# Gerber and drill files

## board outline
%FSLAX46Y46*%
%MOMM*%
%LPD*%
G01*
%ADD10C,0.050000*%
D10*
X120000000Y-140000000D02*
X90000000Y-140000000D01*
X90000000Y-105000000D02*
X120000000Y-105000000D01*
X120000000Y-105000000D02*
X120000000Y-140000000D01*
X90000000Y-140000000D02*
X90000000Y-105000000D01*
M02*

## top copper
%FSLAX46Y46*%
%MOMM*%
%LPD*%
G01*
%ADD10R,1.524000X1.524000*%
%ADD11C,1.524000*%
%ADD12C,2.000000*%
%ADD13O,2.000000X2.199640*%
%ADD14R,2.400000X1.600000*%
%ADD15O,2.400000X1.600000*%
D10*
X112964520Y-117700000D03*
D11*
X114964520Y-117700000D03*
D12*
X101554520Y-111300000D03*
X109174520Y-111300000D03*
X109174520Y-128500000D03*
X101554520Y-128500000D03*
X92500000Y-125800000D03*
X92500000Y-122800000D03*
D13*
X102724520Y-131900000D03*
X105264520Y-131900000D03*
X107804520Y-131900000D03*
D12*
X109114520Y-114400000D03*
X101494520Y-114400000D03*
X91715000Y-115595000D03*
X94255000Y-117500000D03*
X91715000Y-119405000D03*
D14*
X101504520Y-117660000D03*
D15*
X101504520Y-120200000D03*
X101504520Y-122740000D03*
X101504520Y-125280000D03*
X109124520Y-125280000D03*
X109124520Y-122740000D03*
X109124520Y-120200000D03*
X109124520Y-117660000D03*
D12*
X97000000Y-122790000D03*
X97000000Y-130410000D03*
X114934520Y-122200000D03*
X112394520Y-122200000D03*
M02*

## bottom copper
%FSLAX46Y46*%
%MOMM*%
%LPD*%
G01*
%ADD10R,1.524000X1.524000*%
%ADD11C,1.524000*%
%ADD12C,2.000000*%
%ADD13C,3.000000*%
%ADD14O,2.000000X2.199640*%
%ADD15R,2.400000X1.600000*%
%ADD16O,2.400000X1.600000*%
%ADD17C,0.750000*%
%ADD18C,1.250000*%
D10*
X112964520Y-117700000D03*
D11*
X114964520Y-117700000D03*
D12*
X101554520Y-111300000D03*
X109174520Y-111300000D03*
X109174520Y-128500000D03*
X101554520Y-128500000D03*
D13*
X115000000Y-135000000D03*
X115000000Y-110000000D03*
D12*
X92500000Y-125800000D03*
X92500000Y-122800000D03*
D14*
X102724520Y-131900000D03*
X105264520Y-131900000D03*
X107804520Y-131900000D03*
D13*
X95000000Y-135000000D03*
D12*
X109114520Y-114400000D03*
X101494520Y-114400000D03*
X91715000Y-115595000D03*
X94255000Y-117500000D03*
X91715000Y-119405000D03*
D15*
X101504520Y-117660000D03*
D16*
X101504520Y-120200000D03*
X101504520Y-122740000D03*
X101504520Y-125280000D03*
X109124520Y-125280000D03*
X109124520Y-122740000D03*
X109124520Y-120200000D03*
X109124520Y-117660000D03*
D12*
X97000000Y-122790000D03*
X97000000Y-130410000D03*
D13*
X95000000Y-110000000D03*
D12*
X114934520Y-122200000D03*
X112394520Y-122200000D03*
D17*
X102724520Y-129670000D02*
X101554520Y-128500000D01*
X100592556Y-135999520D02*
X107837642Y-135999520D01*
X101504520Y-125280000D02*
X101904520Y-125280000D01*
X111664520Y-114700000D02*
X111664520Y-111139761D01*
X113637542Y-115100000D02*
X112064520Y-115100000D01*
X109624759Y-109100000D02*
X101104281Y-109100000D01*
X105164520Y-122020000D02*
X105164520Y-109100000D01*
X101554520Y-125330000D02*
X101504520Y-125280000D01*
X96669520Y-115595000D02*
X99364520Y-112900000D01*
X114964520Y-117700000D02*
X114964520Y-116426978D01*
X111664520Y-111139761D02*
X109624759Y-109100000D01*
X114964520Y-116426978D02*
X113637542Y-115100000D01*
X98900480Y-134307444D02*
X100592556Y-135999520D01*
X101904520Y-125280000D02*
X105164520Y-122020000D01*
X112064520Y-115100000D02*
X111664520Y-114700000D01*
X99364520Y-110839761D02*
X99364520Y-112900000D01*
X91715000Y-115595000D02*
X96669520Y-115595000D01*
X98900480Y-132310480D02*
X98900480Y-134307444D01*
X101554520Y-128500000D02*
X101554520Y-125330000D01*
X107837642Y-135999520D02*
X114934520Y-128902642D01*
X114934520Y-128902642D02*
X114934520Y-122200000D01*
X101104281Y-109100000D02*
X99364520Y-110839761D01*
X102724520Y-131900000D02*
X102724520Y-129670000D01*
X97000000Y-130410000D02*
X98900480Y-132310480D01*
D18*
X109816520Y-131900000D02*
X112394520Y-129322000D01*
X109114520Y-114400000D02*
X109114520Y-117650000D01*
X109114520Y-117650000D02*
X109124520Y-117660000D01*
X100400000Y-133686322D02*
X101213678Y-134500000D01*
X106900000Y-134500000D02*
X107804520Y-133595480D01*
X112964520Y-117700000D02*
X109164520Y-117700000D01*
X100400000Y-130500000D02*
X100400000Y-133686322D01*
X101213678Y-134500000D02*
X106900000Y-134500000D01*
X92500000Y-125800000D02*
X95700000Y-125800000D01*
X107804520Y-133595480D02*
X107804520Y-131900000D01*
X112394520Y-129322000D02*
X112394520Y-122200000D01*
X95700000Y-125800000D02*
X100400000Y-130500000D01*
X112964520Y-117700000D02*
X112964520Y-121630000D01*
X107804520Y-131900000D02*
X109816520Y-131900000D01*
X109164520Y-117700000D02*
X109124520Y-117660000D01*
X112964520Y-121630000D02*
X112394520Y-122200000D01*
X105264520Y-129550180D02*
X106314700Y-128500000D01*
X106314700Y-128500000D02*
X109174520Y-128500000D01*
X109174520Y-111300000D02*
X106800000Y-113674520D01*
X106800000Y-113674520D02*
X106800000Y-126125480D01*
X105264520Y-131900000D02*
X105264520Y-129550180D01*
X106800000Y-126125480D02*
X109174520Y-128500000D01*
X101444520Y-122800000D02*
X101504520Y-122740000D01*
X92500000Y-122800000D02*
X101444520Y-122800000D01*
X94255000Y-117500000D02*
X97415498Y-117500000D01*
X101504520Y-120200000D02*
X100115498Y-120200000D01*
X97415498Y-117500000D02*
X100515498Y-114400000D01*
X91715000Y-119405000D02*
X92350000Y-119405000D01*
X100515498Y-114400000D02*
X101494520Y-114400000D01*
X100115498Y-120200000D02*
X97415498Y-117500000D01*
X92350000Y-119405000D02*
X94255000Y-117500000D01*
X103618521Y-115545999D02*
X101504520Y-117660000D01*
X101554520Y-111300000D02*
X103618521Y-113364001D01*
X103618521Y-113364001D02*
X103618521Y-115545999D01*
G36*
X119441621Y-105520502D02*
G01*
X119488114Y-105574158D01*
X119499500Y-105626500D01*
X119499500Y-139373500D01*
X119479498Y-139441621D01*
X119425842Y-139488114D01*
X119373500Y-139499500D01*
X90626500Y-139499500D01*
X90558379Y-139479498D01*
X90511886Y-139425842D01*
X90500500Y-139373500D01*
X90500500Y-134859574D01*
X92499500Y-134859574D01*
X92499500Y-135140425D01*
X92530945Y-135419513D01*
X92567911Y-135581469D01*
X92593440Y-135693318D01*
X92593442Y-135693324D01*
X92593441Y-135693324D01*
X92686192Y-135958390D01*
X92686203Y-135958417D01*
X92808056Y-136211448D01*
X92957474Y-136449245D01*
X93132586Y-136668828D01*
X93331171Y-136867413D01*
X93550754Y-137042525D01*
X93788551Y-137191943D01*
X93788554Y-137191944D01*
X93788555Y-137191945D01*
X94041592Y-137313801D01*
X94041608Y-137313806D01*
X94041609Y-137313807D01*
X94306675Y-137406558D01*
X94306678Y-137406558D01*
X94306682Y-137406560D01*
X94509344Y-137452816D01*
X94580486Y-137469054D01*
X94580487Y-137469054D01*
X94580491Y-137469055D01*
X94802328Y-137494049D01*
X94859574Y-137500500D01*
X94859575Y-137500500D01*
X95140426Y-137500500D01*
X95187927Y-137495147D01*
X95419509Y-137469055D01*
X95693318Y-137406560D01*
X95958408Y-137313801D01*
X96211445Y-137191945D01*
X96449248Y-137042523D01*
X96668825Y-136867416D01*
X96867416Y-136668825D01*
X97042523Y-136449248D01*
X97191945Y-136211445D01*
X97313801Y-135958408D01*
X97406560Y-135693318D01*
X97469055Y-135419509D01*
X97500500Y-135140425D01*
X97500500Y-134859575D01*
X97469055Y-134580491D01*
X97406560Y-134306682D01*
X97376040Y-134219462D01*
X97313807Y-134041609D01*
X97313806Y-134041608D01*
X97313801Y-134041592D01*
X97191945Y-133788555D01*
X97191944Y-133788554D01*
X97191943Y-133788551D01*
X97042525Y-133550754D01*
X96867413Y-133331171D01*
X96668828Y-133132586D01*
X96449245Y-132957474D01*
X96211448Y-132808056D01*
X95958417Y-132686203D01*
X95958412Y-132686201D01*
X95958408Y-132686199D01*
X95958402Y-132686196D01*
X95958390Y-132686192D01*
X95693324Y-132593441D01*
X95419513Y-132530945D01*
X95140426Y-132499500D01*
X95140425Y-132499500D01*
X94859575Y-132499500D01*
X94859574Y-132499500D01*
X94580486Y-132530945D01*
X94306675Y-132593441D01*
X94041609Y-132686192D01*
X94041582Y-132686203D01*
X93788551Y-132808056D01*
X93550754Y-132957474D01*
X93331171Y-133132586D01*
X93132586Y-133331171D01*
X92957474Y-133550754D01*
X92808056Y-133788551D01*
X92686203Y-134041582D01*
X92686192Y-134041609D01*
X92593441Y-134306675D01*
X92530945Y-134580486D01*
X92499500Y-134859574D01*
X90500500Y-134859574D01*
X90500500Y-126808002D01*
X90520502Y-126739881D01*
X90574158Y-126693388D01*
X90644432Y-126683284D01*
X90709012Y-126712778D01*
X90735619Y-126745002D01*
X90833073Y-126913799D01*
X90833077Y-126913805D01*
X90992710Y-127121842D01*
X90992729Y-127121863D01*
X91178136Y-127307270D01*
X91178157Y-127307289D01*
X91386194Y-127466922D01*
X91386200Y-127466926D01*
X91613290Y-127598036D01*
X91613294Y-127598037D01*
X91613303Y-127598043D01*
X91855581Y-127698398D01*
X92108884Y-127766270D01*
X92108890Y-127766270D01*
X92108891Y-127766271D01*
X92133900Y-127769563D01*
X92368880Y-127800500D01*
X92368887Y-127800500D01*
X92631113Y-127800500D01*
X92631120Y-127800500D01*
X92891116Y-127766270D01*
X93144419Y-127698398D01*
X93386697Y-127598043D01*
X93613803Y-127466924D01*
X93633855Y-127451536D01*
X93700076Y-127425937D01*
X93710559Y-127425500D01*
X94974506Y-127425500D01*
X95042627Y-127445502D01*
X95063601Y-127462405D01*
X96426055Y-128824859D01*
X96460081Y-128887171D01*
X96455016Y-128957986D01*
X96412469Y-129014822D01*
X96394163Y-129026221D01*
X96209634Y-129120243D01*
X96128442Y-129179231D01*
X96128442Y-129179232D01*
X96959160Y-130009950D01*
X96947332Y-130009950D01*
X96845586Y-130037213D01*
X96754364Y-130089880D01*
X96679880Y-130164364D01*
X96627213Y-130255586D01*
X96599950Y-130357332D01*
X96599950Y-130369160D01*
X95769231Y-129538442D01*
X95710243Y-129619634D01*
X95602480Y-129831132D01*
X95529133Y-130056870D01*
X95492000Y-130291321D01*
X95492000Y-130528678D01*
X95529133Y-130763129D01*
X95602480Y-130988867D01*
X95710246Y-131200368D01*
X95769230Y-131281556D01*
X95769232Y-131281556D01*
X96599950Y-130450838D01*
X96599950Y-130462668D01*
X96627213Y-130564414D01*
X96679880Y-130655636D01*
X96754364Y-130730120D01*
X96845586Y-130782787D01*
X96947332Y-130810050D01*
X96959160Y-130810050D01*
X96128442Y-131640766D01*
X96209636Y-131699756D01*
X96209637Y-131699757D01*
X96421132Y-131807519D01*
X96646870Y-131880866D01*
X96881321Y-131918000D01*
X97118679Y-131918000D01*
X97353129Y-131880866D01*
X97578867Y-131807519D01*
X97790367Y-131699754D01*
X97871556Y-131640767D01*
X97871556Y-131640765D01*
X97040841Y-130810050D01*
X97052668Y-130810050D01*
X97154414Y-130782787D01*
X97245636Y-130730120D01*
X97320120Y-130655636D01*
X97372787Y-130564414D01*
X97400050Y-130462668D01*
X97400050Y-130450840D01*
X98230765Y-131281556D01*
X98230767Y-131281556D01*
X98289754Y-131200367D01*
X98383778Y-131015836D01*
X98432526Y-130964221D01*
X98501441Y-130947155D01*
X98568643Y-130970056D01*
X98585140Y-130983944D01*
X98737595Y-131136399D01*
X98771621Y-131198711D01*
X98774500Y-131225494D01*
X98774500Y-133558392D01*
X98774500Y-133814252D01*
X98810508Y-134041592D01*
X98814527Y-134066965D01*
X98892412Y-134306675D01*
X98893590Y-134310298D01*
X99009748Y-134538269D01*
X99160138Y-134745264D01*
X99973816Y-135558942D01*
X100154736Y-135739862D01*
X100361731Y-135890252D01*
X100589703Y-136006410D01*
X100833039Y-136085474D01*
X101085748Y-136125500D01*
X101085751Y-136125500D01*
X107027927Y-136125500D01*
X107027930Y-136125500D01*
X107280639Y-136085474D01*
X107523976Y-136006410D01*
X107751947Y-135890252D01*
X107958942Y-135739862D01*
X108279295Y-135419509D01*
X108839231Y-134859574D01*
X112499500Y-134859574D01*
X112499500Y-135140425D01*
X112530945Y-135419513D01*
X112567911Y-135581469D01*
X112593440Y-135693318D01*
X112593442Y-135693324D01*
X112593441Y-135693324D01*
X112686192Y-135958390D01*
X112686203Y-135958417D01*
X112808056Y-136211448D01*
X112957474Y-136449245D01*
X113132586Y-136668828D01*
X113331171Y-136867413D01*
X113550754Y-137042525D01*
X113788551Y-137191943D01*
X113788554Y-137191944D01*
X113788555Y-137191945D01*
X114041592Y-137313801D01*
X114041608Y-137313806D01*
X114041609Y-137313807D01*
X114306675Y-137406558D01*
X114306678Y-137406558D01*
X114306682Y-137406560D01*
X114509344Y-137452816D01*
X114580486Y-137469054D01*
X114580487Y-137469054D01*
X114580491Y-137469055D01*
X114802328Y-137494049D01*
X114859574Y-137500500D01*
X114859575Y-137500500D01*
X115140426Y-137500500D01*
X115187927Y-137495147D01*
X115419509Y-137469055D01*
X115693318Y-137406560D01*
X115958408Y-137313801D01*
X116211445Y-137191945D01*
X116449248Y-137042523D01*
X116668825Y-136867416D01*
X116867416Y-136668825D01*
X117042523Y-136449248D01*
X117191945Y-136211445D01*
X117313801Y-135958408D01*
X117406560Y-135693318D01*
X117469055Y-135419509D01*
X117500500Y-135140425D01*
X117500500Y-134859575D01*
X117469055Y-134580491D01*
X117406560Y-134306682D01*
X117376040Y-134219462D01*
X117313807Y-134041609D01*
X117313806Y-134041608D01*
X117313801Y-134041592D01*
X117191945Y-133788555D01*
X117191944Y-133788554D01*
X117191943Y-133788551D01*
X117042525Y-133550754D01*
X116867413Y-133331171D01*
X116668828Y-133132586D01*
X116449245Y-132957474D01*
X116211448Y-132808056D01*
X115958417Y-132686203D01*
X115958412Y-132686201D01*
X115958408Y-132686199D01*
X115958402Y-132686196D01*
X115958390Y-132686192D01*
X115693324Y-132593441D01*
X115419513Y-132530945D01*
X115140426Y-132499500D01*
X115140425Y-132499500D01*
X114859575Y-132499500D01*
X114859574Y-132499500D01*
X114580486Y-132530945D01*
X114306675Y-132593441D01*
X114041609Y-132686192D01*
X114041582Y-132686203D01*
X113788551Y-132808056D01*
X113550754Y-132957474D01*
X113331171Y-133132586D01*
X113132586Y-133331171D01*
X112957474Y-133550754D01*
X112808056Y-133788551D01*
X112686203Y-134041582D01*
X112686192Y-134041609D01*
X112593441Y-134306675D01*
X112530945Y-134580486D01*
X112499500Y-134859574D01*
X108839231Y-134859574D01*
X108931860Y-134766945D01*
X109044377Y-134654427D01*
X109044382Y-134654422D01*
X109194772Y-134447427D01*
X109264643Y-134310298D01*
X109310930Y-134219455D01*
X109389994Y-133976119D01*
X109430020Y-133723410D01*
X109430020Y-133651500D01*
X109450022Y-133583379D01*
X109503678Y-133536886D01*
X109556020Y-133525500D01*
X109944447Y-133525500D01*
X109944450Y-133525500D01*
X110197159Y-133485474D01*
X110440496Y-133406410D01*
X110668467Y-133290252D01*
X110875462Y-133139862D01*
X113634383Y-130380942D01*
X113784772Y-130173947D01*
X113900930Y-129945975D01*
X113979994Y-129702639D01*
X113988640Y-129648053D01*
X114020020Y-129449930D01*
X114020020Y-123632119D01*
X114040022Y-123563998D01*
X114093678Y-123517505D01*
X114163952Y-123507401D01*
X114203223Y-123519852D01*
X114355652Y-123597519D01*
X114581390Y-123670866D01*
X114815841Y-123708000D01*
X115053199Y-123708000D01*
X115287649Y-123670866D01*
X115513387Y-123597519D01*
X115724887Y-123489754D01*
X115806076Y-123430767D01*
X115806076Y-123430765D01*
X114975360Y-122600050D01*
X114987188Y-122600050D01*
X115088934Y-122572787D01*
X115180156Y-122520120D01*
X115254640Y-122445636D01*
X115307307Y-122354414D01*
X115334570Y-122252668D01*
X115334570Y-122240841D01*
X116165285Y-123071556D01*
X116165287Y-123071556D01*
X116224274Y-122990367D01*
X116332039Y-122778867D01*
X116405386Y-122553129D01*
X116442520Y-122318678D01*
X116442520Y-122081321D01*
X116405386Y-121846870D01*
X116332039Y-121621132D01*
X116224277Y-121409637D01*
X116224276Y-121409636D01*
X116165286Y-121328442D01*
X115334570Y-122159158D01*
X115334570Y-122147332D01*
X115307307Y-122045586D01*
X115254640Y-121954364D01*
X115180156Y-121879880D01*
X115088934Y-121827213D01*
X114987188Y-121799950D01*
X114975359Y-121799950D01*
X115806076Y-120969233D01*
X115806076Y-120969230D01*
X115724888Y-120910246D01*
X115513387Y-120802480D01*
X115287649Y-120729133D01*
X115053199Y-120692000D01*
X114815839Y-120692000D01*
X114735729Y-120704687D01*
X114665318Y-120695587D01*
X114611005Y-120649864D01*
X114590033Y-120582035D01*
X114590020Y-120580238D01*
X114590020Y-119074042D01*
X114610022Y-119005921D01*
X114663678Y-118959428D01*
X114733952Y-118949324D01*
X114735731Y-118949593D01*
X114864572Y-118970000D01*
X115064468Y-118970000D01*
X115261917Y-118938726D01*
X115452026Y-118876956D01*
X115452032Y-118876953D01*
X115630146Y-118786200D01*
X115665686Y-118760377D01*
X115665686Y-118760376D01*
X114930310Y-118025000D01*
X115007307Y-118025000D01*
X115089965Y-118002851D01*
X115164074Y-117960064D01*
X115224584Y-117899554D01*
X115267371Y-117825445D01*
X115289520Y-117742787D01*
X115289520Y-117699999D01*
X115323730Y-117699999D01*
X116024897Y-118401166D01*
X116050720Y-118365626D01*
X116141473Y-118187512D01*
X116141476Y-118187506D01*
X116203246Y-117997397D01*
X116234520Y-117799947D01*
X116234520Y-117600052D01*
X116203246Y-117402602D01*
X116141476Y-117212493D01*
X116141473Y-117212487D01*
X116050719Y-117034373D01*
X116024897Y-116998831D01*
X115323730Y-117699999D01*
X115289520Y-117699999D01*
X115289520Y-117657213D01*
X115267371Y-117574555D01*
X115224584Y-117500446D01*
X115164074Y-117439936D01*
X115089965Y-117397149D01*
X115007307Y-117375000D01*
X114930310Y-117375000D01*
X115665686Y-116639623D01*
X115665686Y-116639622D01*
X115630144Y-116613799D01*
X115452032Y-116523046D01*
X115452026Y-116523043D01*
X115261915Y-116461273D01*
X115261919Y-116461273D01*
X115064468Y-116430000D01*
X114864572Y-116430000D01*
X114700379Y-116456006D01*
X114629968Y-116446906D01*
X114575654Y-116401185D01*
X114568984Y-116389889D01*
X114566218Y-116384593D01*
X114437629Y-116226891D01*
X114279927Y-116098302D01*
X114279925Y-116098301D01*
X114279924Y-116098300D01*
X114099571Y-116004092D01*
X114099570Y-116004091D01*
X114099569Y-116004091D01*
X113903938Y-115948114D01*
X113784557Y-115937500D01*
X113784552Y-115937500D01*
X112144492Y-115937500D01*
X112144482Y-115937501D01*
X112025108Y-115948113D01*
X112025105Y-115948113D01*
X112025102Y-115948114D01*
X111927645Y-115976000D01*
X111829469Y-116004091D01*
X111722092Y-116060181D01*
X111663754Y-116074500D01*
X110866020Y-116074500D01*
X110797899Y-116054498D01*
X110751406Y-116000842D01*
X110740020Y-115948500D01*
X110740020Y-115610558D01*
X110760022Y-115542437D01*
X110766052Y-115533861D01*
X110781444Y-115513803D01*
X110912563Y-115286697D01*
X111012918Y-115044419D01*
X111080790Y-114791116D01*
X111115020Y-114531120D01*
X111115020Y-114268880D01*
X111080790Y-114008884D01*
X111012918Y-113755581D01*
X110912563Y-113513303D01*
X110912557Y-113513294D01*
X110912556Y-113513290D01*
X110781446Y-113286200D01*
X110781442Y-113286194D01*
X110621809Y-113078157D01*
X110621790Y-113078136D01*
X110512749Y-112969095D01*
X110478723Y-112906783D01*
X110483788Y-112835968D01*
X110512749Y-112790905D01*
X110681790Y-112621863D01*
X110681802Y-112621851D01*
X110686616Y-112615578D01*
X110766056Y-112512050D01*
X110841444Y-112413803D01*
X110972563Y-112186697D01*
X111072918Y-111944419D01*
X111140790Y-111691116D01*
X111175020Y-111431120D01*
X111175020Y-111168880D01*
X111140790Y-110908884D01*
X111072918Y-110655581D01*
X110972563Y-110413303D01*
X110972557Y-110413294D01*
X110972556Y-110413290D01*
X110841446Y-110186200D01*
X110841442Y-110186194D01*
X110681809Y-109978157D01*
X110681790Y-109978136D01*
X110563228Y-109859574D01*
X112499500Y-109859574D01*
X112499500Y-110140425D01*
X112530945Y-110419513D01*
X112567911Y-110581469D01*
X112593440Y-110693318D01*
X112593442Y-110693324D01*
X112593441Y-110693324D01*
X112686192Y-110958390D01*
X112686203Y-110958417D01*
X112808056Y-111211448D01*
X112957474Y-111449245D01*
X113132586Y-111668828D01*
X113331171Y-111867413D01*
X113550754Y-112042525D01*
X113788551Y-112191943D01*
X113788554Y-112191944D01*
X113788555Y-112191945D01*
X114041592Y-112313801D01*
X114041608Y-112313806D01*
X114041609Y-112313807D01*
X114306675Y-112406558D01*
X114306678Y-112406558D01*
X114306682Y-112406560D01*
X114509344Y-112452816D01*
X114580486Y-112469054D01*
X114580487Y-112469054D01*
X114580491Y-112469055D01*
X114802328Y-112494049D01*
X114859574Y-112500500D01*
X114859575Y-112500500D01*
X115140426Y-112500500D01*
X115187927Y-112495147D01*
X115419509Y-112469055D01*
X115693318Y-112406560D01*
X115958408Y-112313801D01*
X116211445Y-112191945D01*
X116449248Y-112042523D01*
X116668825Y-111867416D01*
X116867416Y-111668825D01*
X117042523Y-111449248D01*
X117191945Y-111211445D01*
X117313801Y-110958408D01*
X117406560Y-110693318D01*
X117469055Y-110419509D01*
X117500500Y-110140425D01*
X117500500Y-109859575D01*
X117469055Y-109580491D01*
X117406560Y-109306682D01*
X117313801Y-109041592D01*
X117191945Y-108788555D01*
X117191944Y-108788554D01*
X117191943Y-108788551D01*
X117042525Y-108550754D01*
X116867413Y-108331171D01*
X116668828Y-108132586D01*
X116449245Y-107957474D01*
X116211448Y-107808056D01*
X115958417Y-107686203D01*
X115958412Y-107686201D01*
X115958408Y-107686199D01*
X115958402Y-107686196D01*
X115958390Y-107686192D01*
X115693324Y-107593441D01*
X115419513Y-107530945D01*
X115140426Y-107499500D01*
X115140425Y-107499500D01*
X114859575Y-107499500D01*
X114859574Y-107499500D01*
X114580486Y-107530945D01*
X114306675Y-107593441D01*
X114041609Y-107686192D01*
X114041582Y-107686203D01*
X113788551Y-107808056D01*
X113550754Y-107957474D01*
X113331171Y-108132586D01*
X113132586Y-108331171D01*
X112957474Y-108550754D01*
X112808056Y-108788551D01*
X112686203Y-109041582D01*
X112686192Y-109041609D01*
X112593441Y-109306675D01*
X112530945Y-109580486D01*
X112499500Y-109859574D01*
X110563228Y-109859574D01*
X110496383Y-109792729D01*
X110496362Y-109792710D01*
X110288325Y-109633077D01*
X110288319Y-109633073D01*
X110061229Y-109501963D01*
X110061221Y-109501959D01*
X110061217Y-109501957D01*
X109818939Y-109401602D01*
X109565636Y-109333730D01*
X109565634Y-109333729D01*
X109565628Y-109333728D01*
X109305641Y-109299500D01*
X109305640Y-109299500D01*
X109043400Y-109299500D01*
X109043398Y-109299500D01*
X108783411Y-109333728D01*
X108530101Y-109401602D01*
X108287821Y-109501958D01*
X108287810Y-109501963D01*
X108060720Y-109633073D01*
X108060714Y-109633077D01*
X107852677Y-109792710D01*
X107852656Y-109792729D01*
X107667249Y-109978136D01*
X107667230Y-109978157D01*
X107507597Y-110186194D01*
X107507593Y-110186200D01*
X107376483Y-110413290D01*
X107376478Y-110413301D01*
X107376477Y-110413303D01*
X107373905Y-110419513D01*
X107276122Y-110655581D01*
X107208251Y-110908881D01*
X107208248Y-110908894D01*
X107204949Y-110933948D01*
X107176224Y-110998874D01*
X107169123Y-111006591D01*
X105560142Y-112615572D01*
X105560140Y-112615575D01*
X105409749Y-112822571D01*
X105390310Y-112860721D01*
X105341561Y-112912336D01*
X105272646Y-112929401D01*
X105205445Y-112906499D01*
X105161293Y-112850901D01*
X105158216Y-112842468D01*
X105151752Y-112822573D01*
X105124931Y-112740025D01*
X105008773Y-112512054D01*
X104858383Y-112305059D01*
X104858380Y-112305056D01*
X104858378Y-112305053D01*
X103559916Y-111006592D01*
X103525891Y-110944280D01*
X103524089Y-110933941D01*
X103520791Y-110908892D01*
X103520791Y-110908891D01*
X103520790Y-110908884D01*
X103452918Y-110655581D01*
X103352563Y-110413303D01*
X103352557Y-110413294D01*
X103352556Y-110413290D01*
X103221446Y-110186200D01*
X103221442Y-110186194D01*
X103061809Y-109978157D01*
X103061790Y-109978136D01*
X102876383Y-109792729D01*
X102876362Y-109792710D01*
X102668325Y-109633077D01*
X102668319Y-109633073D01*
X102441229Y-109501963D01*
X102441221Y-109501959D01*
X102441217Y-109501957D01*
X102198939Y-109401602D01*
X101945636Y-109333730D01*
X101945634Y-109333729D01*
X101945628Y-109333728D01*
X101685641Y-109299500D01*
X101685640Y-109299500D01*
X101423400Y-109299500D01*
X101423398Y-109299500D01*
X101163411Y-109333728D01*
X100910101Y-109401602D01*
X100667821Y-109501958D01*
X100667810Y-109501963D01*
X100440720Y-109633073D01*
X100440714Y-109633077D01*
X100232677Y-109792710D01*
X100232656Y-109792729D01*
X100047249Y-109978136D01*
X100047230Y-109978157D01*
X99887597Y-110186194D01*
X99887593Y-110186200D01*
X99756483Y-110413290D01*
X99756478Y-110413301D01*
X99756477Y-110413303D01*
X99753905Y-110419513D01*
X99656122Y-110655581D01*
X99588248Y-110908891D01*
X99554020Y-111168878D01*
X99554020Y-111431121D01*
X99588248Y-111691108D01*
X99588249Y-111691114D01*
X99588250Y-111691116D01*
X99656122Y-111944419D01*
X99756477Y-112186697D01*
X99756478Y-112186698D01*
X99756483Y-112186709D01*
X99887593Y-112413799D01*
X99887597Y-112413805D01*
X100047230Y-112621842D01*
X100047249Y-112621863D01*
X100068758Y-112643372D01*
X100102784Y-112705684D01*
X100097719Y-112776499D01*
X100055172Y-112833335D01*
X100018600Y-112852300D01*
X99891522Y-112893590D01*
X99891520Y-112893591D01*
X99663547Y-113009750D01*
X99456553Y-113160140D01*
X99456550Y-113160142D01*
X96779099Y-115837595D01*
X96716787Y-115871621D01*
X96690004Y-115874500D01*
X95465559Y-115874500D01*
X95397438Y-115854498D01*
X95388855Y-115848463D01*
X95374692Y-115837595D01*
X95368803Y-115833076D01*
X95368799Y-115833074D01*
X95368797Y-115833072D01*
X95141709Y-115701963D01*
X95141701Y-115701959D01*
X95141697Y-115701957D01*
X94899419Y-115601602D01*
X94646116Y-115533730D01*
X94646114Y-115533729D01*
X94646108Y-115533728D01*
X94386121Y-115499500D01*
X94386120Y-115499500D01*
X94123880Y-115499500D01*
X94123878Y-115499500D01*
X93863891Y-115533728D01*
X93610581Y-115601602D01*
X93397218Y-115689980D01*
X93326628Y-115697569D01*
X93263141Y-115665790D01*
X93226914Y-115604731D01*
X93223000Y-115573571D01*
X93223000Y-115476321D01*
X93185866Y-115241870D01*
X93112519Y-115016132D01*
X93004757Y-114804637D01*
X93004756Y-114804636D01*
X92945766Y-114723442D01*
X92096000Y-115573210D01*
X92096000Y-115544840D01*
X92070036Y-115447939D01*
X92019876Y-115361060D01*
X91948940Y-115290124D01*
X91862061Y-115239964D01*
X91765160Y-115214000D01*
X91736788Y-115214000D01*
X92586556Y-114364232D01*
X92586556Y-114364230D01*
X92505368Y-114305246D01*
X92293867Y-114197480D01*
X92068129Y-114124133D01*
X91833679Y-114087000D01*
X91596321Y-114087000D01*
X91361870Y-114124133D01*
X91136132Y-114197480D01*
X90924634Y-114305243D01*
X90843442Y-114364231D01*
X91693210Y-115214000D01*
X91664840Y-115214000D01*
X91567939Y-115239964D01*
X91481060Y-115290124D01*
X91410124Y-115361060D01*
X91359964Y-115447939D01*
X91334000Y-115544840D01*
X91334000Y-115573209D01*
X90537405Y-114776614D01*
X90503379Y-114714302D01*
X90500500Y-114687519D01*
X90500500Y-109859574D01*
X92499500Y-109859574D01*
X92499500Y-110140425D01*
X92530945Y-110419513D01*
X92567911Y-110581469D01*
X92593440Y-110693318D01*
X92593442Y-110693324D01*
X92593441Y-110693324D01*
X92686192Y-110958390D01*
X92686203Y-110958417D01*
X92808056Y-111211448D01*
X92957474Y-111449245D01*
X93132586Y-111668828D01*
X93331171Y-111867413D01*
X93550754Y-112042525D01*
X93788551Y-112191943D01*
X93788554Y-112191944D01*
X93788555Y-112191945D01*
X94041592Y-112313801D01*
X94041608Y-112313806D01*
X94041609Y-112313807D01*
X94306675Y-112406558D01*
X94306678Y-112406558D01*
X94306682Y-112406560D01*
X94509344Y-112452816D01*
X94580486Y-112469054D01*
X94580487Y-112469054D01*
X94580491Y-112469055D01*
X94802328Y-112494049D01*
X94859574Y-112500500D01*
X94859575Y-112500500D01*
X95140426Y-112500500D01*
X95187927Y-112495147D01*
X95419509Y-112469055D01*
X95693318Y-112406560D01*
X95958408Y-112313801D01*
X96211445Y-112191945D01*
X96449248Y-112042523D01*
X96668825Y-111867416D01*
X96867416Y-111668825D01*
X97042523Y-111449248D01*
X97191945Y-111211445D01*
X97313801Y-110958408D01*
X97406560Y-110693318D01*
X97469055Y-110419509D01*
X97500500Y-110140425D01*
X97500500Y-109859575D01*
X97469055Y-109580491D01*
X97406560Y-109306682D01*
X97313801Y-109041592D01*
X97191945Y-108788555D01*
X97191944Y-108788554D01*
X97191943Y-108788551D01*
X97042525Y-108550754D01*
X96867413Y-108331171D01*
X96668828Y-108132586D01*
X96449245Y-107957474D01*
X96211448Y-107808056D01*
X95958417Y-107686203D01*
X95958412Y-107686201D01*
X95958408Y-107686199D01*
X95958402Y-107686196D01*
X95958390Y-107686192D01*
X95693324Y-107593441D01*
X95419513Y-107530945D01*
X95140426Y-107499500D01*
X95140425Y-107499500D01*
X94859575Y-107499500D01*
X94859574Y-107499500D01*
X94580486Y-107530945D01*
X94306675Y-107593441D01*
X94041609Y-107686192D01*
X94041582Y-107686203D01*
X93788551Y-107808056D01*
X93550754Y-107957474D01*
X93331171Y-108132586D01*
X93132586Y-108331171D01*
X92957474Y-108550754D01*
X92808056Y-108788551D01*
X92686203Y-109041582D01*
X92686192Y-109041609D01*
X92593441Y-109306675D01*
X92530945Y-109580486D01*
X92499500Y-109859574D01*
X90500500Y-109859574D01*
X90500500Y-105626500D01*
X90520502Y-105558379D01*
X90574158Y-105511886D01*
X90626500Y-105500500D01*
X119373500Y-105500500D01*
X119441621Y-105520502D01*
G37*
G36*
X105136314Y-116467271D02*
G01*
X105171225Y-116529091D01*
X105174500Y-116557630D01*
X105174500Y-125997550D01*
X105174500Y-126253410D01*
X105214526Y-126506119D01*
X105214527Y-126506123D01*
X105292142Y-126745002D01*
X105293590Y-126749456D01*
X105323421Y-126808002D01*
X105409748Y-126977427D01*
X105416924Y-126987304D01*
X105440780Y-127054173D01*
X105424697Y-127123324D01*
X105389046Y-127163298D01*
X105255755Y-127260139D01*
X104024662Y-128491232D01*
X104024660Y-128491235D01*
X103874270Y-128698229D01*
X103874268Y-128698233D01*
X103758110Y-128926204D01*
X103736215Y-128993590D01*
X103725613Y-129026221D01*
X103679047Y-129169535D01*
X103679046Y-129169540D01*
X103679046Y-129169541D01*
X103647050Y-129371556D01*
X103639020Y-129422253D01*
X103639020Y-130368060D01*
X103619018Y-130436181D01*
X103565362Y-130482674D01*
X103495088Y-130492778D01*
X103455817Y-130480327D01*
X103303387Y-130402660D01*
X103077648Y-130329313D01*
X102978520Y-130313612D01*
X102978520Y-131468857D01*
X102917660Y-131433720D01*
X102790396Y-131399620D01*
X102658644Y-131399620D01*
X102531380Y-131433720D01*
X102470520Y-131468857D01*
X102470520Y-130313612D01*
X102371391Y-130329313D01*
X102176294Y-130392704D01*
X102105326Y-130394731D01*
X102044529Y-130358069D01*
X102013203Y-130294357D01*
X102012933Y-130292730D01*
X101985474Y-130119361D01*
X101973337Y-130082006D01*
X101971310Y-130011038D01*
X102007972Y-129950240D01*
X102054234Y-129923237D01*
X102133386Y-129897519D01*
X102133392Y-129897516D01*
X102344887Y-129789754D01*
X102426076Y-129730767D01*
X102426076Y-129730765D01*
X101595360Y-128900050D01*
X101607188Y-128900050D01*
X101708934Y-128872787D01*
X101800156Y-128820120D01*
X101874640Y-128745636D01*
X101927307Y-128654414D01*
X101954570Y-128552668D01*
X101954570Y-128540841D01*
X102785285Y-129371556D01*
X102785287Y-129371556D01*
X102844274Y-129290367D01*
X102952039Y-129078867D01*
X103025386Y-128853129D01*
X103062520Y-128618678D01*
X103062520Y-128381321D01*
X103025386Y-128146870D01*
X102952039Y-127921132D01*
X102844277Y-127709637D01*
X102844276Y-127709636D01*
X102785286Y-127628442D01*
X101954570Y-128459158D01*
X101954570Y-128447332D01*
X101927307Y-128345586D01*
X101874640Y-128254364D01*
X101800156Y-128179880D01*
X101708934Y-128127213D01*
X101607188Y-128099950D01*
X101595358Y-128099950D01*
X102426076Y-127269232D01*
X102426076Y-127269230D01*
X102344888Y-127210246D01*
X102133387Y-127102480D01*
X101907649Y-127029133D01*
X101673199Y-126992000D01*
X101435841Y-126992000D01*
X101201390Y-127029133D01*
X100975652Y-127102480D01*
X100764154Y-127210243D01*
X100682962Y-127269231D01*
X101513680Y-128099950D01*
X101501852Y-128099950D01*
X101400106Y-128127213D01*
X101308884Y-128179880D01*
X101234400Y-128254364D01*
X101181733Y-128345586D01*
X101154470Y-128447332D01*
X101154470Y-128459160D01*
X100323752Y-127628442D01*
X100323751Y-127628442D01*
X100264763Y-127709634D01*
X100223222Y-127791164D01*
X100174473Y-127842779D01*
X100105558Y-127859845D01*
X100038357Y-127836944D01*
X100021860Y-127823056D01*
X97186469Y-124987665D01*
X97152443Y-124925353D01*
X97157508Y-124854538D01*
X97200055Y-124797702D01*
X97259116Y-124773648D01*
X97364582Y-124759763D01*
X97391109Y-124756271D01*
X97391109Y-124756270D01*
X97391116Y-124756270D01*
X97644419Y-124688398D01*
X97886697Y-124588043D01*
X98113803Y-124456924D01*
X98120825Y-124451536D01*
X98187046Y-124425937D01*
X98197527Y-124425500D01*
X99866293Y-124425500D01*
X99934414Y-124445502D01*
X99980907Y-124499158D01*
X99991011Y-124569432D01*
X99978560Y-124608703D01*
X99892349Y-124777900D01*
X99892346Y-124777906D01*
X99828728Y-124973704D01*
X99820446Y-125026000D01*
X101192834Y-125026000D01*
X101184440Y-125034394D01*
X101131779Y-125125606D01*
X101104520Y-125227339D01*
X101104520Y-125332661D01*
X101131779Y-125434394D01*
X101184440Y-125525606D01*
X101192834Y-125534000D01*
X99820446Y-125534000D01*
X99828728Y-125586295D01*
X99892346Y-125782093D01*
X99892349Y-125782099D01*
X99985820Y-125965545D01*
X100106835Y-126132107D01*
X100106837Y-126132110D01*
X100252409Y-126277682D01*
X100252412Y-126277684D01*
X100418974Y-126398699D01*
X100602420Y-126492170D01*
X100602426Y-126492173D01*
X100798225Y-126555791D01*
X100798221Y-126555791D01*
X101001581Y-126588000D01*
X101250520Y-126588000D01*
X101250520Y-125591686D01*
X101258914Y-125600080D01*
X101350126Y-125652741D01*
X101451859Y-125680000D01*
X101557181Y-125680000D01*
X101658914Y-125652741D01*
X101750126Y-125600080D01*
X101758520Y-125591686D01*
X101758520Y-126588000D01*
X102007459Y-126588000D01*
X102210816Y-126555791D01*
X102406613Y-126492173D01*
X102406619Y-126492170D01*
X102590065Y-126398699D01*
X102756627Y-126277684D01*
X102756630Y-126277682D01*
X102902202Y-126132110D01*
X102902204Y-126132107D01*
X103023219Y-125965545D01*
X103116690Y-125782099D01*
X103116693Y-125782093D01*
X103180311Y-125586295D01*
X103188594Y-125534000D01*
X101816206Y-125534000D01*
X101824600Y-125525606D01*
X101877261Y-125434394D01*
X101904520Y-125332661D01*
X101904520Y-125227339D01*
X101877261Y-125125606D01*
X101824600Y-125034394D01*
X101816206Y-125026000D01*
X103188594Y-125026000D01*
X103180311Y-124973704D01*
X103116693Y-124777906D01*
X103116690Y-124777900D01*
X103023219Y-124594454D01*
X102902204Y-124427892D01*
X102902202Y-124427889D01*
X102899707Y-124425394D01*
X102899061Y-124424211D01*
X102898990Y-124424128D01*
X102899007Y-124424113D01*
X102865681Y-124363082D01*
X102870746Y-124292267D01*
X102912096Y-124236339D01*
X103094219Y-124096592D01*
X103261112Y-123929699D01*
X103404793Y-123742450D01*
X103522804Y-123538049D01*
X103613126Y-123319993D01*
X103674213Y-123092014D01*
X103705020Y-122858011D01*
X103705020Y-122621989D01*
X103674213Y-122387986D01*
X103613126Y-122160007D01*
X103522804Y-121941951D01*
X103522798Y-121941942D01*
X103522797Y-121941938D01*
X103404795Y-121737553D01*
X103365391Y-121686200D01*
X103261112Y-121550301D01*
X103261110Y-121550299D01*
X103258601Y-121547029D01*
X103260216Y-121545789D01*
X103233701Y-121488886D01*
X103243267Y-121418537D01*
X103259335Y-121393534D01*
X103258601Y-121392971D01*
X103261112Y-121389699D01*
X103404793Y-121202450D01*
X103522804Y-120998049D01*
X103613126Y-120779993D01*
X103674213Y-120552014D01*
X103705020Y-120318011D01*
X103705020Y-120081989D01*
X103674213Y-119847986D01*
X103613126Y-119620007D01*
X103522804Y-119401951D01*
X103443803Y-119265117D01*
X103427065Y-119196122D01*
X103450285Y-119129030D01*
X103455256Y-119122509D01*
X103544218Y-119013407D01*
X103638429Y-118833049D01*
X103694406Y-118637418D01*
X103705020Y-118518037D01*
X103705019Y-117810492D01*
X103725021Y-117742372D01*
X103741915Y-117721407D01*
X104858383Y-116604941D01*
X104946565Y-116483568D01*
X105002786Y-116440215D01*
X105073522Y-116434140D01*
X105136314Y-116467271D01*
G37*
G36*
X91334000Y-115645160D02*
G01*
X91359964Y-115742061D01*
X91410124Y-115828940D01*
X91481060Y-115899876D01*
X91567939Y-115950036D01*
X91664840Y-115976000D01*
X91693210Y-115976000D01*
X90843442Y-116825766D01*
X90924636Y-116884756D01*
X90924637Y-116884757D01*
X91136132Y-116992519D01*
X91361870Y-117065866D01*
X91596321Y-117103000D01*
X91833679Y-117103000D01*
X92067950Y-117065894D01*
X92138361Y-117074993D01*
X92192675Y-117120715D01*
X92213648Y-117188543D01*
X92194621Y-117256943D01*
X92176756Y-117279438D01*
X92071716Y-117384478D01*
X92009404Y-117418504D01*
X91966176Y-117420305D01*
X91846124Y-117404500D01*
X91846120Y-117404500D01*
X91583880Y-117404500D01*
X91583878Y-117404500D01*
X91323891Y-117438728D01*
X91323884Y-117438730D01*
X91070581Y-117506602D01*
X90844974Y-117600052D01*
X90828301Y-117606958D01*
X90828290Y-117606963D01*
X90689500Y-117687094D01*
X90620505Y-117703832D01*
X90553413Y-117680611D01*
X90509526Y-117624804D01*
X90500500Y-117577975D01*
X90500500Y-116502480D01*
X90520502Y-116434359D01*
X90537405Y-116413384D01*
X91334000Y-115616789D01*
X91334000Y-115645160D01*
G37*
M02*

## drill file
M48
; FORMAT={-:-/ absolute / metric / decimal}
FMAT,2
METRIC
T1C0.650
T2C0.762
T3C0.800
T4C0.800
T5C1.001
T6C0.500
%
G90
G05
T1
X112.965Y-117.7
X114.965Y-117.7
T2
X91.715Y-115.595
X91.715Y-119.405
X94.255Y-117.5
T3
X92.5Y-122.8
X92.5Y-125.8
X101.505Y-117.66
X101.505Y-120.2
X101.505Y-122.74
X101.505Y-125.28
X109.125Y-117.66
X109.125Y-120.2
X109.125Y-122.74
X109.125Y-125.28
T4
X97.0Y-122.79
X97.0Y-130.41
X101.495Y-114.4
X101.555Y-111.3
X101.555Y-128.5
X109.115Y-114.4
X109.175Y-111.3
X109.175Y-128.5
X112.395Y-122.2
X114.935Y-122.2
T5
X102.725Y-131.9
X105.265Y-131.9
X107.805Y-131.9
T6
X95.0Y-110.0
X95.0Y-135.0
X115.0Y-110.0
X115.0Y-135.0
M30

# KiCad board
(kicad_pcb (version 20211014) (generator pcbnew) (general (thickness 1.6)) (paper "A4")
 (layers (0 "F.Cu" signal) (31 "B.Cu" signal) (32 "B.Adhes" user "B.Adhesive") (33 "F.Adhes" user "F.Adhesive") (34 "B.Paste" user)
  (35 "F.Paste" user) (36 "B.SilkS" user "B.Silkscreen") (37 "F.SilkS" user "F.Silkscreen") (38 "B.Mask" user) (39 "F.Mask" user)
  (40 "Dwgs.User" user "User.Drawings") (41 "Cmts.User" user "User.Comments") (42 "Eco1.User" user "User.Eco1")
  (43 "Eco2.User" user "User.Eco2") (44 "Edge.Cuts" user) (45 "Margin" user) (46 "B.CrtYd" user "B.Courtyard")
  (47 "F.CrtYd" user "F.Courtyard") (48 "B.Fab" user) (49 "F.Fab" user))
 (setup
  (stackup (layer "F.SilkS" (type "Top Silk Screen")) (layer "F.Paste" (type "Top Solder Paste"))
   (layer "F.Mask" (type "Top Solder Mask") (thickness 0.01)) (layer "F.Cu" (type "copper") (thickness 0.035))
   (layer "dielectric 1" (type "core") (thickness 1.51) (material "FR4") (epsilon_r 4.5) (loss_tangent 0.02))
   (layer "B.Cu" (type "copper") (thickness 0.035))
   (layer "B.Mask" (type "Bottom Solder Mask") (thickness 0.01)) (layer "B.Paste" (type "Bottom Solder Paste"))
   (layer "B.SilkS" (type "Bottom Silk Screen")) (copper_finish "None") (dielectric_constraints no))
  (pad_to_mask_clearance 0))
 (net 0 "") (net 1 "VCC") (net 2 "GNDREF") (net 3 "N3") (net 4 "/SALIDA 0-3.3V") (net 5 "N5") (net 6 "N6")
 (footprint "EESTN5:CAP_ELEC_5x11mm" (layer "F.Cu") (at 113.96452 117.7 -90)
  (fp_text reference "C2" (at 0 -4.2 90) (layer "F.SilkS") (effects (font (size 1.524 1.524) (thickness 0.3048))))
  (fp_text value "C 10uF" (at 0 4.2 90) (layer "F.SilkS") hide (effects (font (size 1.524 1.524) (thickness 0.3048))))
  (pad "1" thru_hole rect locked (at 0 1 270) (size 1.524 1.524) (drill 0.65) (layers *.Cu *.Mask "F.SilkS") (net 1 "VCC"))
  (pad "2" thru_hole circle locked (at 0 -1 270) (size 1.524 1.524) (drill 0.65) (layers *.Cu *.Mask "F.SilkS") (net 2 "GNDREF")))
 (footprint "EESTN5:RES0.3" (layer "F.Cu") (at 105.36452 111.3) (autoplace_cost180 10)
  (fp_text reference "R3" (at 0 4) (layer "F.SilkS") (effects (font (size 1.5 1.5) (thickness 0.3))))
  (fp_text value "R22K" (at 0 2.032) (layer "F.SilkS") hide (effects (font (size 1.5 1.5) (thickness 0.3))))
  (pad "1" thru_hole circle locked (at -3.81 0) (size 2 2) (drill 0.8001) (layers *.Cu *.Mask "F.SilkS") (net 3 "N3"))
  (pad "2" thru_hole circle locked (at 3.81 0) (size 2 2) (drill 0.8001) (layers *.Cu *.Mask "F.SilkS") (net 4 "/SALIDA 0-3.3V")))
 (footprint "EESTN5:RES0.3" (layer "F.Cu") (at 105.36452 128.5 180) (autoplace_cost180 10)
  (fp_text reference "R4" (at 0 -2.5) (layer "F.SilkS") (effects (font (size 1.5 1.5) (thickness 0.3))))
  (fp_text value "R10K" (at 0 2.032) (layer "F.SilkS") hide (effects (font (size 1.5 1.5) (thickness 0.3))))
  (pad "1" thru_hole circle locked (at -3.81 0 180) (size 2 2) (drill 0.8001) (layers *.Cu *.Mask "F.SilkS") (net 4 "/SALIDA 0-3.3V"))
  (pad "2" thru_hole circle locked (at 3.81 0 180) (size 2 2) (drill 0.8001) (layers *.Cu *.Mask "F.SilkS") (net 2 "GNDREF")))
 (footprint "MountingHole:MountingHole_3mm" (layer "F.Cu") (at 115 135)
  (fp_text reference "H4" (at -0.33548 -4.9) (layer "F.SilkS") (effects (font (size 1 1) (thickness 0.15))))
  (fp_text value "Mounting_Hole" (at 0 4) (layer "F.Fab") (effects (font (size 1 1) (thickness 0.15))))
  (pad "" np_thru_hole circle (at 0 0) (size 3 3) (drill 0.5) (layers "B.Cu")))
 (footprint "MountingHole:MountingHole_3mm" (layer "F.Cu") (at 115 110)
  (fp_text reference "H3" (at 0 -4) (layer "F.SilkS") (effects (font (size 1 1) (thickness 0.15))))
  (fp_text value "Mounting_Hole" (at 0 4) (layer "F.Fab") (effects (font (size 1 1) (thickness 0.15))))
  (pad "" np_thru_hole circle (at 0 0) (size 3 3) (drill 0.5) (layers "B.Cu")))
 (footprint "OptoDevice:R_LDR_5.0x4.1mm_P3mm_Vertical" (layer "F.Cu") (at 92.5 125.8 90)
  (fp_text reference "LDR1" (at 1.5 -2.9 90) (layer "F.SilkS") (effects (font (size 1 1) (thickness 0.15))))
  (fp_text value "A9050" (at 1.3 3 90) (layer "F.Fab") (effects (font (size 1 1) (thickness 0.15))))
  (pad "1" thru_hole circle (at 0 0 90) (size 2 2) (drill 0.8) (layers *.Cu *.Mask) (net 1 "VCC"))
  (pad "2" thru_hole circle (at 3 0 90) (size 2 2) (drill 0.8) (layers *.Cu *.Mask) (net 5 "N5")))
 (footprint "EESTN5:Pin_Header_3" (layer "F.Cu") (at 105.26452 131.9)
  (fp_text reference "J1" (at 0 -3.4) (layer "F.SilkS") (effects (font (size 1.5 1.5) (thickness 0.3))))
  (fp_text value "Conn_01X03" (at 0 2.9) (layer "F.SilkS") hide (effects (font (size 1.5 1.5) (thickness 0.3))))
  (pad "1" thru_hole oval locked (at -2.54 0) (size 2 2.19964) (drill 1.00076) (layers *.Cu *.Mask "F.SilkS") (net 2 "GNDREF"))
  (pad "2" thru_hole oval locked (at 0 0) (size 2 2.19964) (drill 1.00076) (layers *.Cu *.Mask "F.SilkS") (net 4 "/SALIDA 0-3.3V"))
  (pad "3" thru_hole oval locked (at 2.54 0) (size 2 2.19964) (drill 1.00076) (layers *.Cu *.Mask "F.SilkS") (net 1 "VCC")))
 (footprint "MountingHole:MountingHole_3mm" (layer "F.Cu") (at 95 135)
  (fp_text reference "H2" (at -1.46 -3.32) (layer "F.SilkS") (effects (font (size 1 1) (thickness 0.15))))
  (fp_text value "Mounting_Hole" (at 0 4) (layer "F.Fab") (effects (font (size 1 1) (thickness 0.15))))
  (pad "" np_thru_hole circle (at 0 0) (size 3 3) (drill 0.5) (layers "B.Cu")))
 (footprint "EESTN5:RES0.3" (layer "F.Cu") (at 105.30452 114.4 180) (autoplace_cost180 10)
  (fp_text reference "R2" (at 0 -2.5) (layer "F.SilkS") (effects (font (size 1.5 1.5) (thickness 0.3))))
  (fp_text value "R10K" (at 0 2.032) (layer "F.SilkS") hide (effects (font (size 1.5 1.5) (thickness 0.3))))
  (pad "1" thru_hole circle locked (at -3.81 0 180) (size 2 2) (drill 0.8001) (layers *.Cu *.Mask "F.SilkS") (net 1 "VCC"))
  (pad "2" thru_hole circle locked (at 3.81 0 180) (size 2 2) (drill 0.8001) (layers *.Cu *.Mask "F.SilkS") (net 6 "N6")))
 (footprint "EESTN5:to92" (layer "F.Cu") (at 92.35 117.5 -90)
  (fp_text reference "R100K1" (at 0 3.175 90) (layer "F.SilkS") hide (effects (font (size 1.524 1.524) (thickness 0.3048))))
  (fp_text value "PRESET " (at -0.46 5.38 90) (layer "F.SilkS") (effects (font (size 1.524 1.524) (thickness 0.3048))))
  (pad "1" thru_hole circle locked (at -1.905 0.635 270) (size 2 2) (drill 0.762) (layers *.Cu *.Mask "F.SilkS") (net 2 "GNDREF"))
  (pad "2" thru_hole circle locked (at 0 -1.905 270) (size 2 2) (drill 0.762) (layers *.Cu *.Mask "F.SilkS") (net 6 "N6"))
  (pad "3" thru_hole circle locked (at 1.905 0.635 270) (size 2 2) (drill 0.762) (layers *.Cu *.Mask "F.SilkS") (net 6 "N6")))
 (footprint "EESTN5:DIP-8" (layer "F.Cu") (at 101.50452 117.66)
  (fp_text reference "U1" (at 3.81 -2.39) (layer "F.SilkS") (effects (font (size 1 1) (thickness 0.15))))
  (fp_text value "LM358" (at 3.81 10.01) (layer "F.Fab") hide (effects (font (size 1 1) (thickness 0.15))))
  (pad "1" thru_hole rect locked (at 0 0) (size 2.4 1.6) (drill 0.8) (layers *.Cu *.Mask) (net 3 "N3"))
  (pad "2" thru_hole oval locked (at 0 2.54) (size 2.4 1.6) (drill 0.8) (layers *.Cu *.Mask) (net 6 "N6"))
  (pad "3" thru_hole oval locked (at 0 5.08) (size 2.4 1.6) (drill 0.8) (layers *.Cu *.Mask) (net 5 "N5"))
  (pad "4" thru_hole oval locked (at 0 7.62) (size 2.4 1.6) (drill 0.8) (layers *.Cu *.Mask) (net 2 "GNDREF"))
  (pad "5" thru_hole oval locked (at 7.62 7.62) (size 2.4 1.6) (drill 0.8) (layers *.Cu *.Mask))
  (pad "6" thru_hole oval locked (at 7.62 5.08) (size 2.4 1.6) (drill 0.8) (layers *.Cu *.Mask))
  (pad "7" thru_hole oval locked (at 7.62 2.54) (size 2.4 1.6) (drill 0.8) (layers *.Cu *.Mask))
  (pad "8" thru_hole oval locked (at 7.62 0) (size 2.4 1.6) (drill 0.8) (layers *.Cu *.Mask) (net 1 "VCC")))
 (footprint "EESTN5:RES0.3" (layer "F.Cu") (at 97 126.6 -90) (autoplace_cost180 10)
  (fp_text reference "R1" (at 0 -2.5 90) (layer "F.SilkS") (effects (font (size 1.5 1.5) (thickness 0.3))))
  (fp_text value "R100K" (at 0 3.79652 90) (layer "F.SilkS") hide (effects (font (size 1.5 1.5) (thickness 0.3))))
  (pad "1" thru_hole circle locked (at -3.81 0 270) (size 2 2) (drill 0.8001) (layers *.Cu *.Mask "F.SilkS") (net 5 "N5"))
  (pad "2" thru_hole circle locked (at 3.81 0 270) (size 2 2) (drill 0.8001) (layers *.Cu *.Mask "F.SilkS") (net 2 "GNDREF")))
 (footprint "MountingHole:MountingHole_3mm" (layer "F.Cu") (at 95 110)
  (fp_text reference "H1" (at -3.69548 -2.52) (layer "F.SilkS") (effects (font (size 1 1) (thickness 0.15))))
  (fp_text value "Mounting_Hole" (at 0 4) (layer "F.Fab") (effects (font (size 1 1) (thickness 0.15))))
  (pad "" np_thru_hole circle (at 0 0) (size 3 3) (drill 0.5) (layers "B.Cu")))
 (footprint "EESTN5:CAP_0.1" (layer "F.Cu") (at 113.66452 122.2 180)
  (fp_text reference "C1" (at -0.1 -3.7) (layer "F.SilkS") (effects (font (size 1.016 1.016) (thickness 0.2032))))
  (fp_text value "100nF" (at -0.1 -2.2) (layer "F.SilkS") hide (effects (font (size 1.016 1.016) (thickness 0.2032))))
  (pad "1" thru_hole circle locked (at -1.27 0 180) (size 2 2) (drill 0.8001) (layers *.Cu *.Mask "F.SilkS") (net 2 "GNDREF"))
  (pad "2" thru_hole circle locked (at 1.27 0 180) (size 2 2) (drill 0.8001) (layers *.Cu *.Mask "F.SilkS") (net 1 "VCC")))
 (gr_line (start 120 140) (end 90 140) (layer "Edge.Cuts") (width 0.05))
 (gr_line (start 90 105) (end 120 105) (layer "Edge.Cuts") (width 0.05))
 (gr_line (start 120 105) (end 120 140) (layer "Edge.Cuts") (width 0.05))
 (gr_line (start 90 140) (end 90 105) (layer "Edge.Cuts") (width 0.05))
 (segment (start 102.72452 129.67) (end 101.55452 128.5) (width 0.75) (layer "B.Cu") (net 2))
 (segment (start 100.592556 135.99952) (end 107.837642 135.99952) (width 0.75) (layer "B.Cu") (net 2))
 (segment (start 101.50452 125.28) (end 101.90452 125.28) (width 0.75) (layer "B.Cu") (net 2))
 (segment (start 111.66452 114.7) (end 111.66452 111.139761) (width 0.75) (layer "B.Cu") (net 2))
 (segment (start 113.637542 115.1) (end 112.06452 115.1) (width 0.75) (layer "B.Cu") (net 2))
 (segment (start 109.624759 109.1) (end 101.104281 109.1) (width 0.75) (layer "B.Cu") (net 2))
 (segment (start 105.16452 122.02) (end 105.16452 109.1) (width 0.75) (layer "B.Cu") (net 2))
 (segment (start 101.55452 125.33) (end 101.50452 125.28) (width 0.75) (layer "B.Cu") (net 2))
 (segment (start 96.66952 115.595) (end 99.36452 112.9) (width 0.75) (layer "B.Cu") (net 2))
 (segment (start 114.96452 117.7) (end 114.96452 116.426978) (width 0.75) (layer "B.Cu") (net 2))
 (segment (start 111.66452 111.139761) (end 109.624759 109.1) (width 0.75) (layer "B.Cu") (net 2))
 (segment (start 114.96452 116.426978) (end 113.637542 115.1) (width 0.75) (layer "B.Cu") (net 2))
 (segment (start 98.90048 134.307444) (end 100.592556 135.99952) (width 0.75) (layer "B.Cu") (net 2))
 (segment (start 101.90452 125.28) (end 105.16452 122.02) (width 0.75) (layer "B.Cu") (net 2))
 (segment (start 112.06452 115.1) (end 111.66452 114.7) (width 0.75) (layer "B.Cu") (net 2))
 (segment (start 99.36452 110.839761) (end 99.36452 112.9) (width 0.75) (layer "B.Cu") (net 2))
 (segment (start 91.715 115.595) (end 96.66952 115.595) (width 0.75) (layer "B.Cu") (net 2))
 (segment (start 98.90048 132.31048) (end 98.90048 134.307444) (width 0.75) (layer "B.Cu") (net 2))
 (segment (start 101.55452 128.5) (end 101.55452 125.33) (width 0.75) (layer "B.Cu") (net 2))
 (segment (start 107.837642 135.99952) (end 114.93452 128.902642) (width 0.75) (layer "B.Cu") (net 2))
 (segment (start 114.93452 128.902642) (end 114.93452 122.2) (width 0.75) (layer "B.Cu") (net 2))
 (segment (start 101.104281 109.1) (end 99.36452 110.839761) (width 0.75) (layer "B.Cu") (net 2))
 (segment (start 102.72452 131.9) (end 102.72452 129.67) (width 0.75) (layer "B.Cu") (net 2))
 (segment (start 97 130.41) (end 98.90048 132.31048) (width 0.75) (layer "B.Cu") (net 2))
 (segment (start 109.81652 131.9) (end 112.39452 129.322) (width 1.25) (layer "B.Cu") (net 1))
 (segment (start 109.11452 114.4) (end 109.11452 117.65) (width 1.25) (layer "B.Cu") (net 1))
 (segment (start 109.11452 117.65) (end 109.12452 117.66) (width 1.25) (layer "B.Cu") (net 1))
 (segment (start 100.4 133.686322) (end 101.213678 134.5) (width 1.25) (layer "B.Cu") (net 1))
 (segment (start 106.9 134.5) (end 107.80452 133.59548) (width 1.25) (layer "B.Cu") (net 1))
 (segment (start 112.96452 117.7) (end 109.16452 117.7) (width 1.25) (layer "B.Cu") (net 1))
 (segment (start 100.4 130.5) (end 100.4 133.686322) (width 1.25) (layer "B.Cu") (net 1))
 (segment (start 101.213678 134.5) (end 106.9 134.5) (width 1.25) (layer "B.Cu") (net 1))
 (segment (start 92.5 125.8) (end 95.7 125.8) (width 1.25) (layer "B.Cu") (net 1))
 (segment (start 107.80452 133.59548) (end 107.80452 131.9) (width 1.25) (layer "B.Cu") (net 1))
 (segment (start 112.39452 129.322) (end 112.39452 122.2) (width 1.25) (layer "B.Cu") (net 1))
 (segment (start 95.7 125.8) (end 100.4 130.5) (width 1.25) (layer "B.Cu") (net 1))
 (segment (start 112.96452 117.7) (end 112.96452 121.63) (width 1.25) (layer "B.Cu") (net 1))
 (segment (start 107.80452 131.9) (end 109.81652 131.9) (width 1.25) (layer "B.Cu") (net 1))
 (segment (start 109.16452 117.7) (end 109.12452 117.66) (width 1.25) (layer "B.Cu") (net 1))
 (segment (start 112.96452 121.63) (end 112.39452 122.2) (width 1.25) (layer "B.Cu") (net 1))
 (segment (start 105.26452 129.55018) (end 106.3147 128.5) (width 1.25) (layer "B.Cu") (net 4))
 (segment (start 106.3147 128.5) (end 109.17452 128.5) (width 1.25) (layer "B.Cu") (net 4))
 (segment (start 109.17452 111.3) (end 106.8 113.67452) (width 1.25) (layer "B.Cu") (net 4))
 (segment (start 106.8 113.67452) (end 106.8 126.12548) (width 1.25) (layer "B.Cu") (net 4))
 (segment (start 105.26452 131.9) (end 105.26452 129.55018) (width 1.25) (layer "B.Cu") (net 4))
 (segment (start 106.8 126.12548) (end 109.17452 128.5) (width 1.25) (layer "B.Cu") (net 4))
 (segment (start 101.44452 122.8) (end 101.50452 122.74) (width 1.25) (layer "B.Cu") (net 5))
 (segment (start 92.5 122.8) (end 101.44452 122.8) (width 1.25) (layer "B.Cu") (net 5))
 (segment (start 94.255 117.5) (end 97.415498 117.5) (width 1.25) (layer "B.Cu") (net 6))
 (segment (start 101.50452 120.2) (end 100.115498 120.2) (width 1.25) (layer "B.Cu") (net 6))
 (segment (start 97.415498 117.5) (end 100.515498 114.4) (width 1.25) (layer "B.Cu") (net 6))
 (segment (start 91.715 119.405) (end 92.35 119.405) (width 1.25) (layer "B.Cu") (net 6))
 (segment (start 100.515498 114.4) (end 101.49452 114.4) (width 1.25) (layer "B.Cu") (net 6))
 (segment (start 100.115498 120.2) (end 97.415498 117.5) (width 1.25) (layer "B.Cu") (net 6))
 (segment (start 92.35 119.405) (end 94.255 117.5) (width 1.25) (layer "B.Cu") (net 6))
 (segment (start 103.618521 115.545999) (end 101.50452 117.66) (width 1.25) (layer "B.Cu") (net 3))
 (segment (start 101.55452 111.3) (end 103.618521 113.364001) (width 1.25) (layer "B.Cu") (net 3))
 (segment (start 103.618521 113.364001) (end 103.618521 115.545999) (width 1.25) (layer "B.Cu") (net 3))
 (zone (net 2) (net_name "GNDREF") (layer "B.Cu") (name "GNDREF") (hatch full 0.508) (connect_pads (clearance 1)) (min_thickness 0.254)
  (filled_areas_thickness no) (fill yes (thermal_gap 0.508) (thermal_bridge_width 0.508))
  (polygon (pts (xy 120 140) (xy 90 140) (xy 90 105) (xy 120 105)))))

